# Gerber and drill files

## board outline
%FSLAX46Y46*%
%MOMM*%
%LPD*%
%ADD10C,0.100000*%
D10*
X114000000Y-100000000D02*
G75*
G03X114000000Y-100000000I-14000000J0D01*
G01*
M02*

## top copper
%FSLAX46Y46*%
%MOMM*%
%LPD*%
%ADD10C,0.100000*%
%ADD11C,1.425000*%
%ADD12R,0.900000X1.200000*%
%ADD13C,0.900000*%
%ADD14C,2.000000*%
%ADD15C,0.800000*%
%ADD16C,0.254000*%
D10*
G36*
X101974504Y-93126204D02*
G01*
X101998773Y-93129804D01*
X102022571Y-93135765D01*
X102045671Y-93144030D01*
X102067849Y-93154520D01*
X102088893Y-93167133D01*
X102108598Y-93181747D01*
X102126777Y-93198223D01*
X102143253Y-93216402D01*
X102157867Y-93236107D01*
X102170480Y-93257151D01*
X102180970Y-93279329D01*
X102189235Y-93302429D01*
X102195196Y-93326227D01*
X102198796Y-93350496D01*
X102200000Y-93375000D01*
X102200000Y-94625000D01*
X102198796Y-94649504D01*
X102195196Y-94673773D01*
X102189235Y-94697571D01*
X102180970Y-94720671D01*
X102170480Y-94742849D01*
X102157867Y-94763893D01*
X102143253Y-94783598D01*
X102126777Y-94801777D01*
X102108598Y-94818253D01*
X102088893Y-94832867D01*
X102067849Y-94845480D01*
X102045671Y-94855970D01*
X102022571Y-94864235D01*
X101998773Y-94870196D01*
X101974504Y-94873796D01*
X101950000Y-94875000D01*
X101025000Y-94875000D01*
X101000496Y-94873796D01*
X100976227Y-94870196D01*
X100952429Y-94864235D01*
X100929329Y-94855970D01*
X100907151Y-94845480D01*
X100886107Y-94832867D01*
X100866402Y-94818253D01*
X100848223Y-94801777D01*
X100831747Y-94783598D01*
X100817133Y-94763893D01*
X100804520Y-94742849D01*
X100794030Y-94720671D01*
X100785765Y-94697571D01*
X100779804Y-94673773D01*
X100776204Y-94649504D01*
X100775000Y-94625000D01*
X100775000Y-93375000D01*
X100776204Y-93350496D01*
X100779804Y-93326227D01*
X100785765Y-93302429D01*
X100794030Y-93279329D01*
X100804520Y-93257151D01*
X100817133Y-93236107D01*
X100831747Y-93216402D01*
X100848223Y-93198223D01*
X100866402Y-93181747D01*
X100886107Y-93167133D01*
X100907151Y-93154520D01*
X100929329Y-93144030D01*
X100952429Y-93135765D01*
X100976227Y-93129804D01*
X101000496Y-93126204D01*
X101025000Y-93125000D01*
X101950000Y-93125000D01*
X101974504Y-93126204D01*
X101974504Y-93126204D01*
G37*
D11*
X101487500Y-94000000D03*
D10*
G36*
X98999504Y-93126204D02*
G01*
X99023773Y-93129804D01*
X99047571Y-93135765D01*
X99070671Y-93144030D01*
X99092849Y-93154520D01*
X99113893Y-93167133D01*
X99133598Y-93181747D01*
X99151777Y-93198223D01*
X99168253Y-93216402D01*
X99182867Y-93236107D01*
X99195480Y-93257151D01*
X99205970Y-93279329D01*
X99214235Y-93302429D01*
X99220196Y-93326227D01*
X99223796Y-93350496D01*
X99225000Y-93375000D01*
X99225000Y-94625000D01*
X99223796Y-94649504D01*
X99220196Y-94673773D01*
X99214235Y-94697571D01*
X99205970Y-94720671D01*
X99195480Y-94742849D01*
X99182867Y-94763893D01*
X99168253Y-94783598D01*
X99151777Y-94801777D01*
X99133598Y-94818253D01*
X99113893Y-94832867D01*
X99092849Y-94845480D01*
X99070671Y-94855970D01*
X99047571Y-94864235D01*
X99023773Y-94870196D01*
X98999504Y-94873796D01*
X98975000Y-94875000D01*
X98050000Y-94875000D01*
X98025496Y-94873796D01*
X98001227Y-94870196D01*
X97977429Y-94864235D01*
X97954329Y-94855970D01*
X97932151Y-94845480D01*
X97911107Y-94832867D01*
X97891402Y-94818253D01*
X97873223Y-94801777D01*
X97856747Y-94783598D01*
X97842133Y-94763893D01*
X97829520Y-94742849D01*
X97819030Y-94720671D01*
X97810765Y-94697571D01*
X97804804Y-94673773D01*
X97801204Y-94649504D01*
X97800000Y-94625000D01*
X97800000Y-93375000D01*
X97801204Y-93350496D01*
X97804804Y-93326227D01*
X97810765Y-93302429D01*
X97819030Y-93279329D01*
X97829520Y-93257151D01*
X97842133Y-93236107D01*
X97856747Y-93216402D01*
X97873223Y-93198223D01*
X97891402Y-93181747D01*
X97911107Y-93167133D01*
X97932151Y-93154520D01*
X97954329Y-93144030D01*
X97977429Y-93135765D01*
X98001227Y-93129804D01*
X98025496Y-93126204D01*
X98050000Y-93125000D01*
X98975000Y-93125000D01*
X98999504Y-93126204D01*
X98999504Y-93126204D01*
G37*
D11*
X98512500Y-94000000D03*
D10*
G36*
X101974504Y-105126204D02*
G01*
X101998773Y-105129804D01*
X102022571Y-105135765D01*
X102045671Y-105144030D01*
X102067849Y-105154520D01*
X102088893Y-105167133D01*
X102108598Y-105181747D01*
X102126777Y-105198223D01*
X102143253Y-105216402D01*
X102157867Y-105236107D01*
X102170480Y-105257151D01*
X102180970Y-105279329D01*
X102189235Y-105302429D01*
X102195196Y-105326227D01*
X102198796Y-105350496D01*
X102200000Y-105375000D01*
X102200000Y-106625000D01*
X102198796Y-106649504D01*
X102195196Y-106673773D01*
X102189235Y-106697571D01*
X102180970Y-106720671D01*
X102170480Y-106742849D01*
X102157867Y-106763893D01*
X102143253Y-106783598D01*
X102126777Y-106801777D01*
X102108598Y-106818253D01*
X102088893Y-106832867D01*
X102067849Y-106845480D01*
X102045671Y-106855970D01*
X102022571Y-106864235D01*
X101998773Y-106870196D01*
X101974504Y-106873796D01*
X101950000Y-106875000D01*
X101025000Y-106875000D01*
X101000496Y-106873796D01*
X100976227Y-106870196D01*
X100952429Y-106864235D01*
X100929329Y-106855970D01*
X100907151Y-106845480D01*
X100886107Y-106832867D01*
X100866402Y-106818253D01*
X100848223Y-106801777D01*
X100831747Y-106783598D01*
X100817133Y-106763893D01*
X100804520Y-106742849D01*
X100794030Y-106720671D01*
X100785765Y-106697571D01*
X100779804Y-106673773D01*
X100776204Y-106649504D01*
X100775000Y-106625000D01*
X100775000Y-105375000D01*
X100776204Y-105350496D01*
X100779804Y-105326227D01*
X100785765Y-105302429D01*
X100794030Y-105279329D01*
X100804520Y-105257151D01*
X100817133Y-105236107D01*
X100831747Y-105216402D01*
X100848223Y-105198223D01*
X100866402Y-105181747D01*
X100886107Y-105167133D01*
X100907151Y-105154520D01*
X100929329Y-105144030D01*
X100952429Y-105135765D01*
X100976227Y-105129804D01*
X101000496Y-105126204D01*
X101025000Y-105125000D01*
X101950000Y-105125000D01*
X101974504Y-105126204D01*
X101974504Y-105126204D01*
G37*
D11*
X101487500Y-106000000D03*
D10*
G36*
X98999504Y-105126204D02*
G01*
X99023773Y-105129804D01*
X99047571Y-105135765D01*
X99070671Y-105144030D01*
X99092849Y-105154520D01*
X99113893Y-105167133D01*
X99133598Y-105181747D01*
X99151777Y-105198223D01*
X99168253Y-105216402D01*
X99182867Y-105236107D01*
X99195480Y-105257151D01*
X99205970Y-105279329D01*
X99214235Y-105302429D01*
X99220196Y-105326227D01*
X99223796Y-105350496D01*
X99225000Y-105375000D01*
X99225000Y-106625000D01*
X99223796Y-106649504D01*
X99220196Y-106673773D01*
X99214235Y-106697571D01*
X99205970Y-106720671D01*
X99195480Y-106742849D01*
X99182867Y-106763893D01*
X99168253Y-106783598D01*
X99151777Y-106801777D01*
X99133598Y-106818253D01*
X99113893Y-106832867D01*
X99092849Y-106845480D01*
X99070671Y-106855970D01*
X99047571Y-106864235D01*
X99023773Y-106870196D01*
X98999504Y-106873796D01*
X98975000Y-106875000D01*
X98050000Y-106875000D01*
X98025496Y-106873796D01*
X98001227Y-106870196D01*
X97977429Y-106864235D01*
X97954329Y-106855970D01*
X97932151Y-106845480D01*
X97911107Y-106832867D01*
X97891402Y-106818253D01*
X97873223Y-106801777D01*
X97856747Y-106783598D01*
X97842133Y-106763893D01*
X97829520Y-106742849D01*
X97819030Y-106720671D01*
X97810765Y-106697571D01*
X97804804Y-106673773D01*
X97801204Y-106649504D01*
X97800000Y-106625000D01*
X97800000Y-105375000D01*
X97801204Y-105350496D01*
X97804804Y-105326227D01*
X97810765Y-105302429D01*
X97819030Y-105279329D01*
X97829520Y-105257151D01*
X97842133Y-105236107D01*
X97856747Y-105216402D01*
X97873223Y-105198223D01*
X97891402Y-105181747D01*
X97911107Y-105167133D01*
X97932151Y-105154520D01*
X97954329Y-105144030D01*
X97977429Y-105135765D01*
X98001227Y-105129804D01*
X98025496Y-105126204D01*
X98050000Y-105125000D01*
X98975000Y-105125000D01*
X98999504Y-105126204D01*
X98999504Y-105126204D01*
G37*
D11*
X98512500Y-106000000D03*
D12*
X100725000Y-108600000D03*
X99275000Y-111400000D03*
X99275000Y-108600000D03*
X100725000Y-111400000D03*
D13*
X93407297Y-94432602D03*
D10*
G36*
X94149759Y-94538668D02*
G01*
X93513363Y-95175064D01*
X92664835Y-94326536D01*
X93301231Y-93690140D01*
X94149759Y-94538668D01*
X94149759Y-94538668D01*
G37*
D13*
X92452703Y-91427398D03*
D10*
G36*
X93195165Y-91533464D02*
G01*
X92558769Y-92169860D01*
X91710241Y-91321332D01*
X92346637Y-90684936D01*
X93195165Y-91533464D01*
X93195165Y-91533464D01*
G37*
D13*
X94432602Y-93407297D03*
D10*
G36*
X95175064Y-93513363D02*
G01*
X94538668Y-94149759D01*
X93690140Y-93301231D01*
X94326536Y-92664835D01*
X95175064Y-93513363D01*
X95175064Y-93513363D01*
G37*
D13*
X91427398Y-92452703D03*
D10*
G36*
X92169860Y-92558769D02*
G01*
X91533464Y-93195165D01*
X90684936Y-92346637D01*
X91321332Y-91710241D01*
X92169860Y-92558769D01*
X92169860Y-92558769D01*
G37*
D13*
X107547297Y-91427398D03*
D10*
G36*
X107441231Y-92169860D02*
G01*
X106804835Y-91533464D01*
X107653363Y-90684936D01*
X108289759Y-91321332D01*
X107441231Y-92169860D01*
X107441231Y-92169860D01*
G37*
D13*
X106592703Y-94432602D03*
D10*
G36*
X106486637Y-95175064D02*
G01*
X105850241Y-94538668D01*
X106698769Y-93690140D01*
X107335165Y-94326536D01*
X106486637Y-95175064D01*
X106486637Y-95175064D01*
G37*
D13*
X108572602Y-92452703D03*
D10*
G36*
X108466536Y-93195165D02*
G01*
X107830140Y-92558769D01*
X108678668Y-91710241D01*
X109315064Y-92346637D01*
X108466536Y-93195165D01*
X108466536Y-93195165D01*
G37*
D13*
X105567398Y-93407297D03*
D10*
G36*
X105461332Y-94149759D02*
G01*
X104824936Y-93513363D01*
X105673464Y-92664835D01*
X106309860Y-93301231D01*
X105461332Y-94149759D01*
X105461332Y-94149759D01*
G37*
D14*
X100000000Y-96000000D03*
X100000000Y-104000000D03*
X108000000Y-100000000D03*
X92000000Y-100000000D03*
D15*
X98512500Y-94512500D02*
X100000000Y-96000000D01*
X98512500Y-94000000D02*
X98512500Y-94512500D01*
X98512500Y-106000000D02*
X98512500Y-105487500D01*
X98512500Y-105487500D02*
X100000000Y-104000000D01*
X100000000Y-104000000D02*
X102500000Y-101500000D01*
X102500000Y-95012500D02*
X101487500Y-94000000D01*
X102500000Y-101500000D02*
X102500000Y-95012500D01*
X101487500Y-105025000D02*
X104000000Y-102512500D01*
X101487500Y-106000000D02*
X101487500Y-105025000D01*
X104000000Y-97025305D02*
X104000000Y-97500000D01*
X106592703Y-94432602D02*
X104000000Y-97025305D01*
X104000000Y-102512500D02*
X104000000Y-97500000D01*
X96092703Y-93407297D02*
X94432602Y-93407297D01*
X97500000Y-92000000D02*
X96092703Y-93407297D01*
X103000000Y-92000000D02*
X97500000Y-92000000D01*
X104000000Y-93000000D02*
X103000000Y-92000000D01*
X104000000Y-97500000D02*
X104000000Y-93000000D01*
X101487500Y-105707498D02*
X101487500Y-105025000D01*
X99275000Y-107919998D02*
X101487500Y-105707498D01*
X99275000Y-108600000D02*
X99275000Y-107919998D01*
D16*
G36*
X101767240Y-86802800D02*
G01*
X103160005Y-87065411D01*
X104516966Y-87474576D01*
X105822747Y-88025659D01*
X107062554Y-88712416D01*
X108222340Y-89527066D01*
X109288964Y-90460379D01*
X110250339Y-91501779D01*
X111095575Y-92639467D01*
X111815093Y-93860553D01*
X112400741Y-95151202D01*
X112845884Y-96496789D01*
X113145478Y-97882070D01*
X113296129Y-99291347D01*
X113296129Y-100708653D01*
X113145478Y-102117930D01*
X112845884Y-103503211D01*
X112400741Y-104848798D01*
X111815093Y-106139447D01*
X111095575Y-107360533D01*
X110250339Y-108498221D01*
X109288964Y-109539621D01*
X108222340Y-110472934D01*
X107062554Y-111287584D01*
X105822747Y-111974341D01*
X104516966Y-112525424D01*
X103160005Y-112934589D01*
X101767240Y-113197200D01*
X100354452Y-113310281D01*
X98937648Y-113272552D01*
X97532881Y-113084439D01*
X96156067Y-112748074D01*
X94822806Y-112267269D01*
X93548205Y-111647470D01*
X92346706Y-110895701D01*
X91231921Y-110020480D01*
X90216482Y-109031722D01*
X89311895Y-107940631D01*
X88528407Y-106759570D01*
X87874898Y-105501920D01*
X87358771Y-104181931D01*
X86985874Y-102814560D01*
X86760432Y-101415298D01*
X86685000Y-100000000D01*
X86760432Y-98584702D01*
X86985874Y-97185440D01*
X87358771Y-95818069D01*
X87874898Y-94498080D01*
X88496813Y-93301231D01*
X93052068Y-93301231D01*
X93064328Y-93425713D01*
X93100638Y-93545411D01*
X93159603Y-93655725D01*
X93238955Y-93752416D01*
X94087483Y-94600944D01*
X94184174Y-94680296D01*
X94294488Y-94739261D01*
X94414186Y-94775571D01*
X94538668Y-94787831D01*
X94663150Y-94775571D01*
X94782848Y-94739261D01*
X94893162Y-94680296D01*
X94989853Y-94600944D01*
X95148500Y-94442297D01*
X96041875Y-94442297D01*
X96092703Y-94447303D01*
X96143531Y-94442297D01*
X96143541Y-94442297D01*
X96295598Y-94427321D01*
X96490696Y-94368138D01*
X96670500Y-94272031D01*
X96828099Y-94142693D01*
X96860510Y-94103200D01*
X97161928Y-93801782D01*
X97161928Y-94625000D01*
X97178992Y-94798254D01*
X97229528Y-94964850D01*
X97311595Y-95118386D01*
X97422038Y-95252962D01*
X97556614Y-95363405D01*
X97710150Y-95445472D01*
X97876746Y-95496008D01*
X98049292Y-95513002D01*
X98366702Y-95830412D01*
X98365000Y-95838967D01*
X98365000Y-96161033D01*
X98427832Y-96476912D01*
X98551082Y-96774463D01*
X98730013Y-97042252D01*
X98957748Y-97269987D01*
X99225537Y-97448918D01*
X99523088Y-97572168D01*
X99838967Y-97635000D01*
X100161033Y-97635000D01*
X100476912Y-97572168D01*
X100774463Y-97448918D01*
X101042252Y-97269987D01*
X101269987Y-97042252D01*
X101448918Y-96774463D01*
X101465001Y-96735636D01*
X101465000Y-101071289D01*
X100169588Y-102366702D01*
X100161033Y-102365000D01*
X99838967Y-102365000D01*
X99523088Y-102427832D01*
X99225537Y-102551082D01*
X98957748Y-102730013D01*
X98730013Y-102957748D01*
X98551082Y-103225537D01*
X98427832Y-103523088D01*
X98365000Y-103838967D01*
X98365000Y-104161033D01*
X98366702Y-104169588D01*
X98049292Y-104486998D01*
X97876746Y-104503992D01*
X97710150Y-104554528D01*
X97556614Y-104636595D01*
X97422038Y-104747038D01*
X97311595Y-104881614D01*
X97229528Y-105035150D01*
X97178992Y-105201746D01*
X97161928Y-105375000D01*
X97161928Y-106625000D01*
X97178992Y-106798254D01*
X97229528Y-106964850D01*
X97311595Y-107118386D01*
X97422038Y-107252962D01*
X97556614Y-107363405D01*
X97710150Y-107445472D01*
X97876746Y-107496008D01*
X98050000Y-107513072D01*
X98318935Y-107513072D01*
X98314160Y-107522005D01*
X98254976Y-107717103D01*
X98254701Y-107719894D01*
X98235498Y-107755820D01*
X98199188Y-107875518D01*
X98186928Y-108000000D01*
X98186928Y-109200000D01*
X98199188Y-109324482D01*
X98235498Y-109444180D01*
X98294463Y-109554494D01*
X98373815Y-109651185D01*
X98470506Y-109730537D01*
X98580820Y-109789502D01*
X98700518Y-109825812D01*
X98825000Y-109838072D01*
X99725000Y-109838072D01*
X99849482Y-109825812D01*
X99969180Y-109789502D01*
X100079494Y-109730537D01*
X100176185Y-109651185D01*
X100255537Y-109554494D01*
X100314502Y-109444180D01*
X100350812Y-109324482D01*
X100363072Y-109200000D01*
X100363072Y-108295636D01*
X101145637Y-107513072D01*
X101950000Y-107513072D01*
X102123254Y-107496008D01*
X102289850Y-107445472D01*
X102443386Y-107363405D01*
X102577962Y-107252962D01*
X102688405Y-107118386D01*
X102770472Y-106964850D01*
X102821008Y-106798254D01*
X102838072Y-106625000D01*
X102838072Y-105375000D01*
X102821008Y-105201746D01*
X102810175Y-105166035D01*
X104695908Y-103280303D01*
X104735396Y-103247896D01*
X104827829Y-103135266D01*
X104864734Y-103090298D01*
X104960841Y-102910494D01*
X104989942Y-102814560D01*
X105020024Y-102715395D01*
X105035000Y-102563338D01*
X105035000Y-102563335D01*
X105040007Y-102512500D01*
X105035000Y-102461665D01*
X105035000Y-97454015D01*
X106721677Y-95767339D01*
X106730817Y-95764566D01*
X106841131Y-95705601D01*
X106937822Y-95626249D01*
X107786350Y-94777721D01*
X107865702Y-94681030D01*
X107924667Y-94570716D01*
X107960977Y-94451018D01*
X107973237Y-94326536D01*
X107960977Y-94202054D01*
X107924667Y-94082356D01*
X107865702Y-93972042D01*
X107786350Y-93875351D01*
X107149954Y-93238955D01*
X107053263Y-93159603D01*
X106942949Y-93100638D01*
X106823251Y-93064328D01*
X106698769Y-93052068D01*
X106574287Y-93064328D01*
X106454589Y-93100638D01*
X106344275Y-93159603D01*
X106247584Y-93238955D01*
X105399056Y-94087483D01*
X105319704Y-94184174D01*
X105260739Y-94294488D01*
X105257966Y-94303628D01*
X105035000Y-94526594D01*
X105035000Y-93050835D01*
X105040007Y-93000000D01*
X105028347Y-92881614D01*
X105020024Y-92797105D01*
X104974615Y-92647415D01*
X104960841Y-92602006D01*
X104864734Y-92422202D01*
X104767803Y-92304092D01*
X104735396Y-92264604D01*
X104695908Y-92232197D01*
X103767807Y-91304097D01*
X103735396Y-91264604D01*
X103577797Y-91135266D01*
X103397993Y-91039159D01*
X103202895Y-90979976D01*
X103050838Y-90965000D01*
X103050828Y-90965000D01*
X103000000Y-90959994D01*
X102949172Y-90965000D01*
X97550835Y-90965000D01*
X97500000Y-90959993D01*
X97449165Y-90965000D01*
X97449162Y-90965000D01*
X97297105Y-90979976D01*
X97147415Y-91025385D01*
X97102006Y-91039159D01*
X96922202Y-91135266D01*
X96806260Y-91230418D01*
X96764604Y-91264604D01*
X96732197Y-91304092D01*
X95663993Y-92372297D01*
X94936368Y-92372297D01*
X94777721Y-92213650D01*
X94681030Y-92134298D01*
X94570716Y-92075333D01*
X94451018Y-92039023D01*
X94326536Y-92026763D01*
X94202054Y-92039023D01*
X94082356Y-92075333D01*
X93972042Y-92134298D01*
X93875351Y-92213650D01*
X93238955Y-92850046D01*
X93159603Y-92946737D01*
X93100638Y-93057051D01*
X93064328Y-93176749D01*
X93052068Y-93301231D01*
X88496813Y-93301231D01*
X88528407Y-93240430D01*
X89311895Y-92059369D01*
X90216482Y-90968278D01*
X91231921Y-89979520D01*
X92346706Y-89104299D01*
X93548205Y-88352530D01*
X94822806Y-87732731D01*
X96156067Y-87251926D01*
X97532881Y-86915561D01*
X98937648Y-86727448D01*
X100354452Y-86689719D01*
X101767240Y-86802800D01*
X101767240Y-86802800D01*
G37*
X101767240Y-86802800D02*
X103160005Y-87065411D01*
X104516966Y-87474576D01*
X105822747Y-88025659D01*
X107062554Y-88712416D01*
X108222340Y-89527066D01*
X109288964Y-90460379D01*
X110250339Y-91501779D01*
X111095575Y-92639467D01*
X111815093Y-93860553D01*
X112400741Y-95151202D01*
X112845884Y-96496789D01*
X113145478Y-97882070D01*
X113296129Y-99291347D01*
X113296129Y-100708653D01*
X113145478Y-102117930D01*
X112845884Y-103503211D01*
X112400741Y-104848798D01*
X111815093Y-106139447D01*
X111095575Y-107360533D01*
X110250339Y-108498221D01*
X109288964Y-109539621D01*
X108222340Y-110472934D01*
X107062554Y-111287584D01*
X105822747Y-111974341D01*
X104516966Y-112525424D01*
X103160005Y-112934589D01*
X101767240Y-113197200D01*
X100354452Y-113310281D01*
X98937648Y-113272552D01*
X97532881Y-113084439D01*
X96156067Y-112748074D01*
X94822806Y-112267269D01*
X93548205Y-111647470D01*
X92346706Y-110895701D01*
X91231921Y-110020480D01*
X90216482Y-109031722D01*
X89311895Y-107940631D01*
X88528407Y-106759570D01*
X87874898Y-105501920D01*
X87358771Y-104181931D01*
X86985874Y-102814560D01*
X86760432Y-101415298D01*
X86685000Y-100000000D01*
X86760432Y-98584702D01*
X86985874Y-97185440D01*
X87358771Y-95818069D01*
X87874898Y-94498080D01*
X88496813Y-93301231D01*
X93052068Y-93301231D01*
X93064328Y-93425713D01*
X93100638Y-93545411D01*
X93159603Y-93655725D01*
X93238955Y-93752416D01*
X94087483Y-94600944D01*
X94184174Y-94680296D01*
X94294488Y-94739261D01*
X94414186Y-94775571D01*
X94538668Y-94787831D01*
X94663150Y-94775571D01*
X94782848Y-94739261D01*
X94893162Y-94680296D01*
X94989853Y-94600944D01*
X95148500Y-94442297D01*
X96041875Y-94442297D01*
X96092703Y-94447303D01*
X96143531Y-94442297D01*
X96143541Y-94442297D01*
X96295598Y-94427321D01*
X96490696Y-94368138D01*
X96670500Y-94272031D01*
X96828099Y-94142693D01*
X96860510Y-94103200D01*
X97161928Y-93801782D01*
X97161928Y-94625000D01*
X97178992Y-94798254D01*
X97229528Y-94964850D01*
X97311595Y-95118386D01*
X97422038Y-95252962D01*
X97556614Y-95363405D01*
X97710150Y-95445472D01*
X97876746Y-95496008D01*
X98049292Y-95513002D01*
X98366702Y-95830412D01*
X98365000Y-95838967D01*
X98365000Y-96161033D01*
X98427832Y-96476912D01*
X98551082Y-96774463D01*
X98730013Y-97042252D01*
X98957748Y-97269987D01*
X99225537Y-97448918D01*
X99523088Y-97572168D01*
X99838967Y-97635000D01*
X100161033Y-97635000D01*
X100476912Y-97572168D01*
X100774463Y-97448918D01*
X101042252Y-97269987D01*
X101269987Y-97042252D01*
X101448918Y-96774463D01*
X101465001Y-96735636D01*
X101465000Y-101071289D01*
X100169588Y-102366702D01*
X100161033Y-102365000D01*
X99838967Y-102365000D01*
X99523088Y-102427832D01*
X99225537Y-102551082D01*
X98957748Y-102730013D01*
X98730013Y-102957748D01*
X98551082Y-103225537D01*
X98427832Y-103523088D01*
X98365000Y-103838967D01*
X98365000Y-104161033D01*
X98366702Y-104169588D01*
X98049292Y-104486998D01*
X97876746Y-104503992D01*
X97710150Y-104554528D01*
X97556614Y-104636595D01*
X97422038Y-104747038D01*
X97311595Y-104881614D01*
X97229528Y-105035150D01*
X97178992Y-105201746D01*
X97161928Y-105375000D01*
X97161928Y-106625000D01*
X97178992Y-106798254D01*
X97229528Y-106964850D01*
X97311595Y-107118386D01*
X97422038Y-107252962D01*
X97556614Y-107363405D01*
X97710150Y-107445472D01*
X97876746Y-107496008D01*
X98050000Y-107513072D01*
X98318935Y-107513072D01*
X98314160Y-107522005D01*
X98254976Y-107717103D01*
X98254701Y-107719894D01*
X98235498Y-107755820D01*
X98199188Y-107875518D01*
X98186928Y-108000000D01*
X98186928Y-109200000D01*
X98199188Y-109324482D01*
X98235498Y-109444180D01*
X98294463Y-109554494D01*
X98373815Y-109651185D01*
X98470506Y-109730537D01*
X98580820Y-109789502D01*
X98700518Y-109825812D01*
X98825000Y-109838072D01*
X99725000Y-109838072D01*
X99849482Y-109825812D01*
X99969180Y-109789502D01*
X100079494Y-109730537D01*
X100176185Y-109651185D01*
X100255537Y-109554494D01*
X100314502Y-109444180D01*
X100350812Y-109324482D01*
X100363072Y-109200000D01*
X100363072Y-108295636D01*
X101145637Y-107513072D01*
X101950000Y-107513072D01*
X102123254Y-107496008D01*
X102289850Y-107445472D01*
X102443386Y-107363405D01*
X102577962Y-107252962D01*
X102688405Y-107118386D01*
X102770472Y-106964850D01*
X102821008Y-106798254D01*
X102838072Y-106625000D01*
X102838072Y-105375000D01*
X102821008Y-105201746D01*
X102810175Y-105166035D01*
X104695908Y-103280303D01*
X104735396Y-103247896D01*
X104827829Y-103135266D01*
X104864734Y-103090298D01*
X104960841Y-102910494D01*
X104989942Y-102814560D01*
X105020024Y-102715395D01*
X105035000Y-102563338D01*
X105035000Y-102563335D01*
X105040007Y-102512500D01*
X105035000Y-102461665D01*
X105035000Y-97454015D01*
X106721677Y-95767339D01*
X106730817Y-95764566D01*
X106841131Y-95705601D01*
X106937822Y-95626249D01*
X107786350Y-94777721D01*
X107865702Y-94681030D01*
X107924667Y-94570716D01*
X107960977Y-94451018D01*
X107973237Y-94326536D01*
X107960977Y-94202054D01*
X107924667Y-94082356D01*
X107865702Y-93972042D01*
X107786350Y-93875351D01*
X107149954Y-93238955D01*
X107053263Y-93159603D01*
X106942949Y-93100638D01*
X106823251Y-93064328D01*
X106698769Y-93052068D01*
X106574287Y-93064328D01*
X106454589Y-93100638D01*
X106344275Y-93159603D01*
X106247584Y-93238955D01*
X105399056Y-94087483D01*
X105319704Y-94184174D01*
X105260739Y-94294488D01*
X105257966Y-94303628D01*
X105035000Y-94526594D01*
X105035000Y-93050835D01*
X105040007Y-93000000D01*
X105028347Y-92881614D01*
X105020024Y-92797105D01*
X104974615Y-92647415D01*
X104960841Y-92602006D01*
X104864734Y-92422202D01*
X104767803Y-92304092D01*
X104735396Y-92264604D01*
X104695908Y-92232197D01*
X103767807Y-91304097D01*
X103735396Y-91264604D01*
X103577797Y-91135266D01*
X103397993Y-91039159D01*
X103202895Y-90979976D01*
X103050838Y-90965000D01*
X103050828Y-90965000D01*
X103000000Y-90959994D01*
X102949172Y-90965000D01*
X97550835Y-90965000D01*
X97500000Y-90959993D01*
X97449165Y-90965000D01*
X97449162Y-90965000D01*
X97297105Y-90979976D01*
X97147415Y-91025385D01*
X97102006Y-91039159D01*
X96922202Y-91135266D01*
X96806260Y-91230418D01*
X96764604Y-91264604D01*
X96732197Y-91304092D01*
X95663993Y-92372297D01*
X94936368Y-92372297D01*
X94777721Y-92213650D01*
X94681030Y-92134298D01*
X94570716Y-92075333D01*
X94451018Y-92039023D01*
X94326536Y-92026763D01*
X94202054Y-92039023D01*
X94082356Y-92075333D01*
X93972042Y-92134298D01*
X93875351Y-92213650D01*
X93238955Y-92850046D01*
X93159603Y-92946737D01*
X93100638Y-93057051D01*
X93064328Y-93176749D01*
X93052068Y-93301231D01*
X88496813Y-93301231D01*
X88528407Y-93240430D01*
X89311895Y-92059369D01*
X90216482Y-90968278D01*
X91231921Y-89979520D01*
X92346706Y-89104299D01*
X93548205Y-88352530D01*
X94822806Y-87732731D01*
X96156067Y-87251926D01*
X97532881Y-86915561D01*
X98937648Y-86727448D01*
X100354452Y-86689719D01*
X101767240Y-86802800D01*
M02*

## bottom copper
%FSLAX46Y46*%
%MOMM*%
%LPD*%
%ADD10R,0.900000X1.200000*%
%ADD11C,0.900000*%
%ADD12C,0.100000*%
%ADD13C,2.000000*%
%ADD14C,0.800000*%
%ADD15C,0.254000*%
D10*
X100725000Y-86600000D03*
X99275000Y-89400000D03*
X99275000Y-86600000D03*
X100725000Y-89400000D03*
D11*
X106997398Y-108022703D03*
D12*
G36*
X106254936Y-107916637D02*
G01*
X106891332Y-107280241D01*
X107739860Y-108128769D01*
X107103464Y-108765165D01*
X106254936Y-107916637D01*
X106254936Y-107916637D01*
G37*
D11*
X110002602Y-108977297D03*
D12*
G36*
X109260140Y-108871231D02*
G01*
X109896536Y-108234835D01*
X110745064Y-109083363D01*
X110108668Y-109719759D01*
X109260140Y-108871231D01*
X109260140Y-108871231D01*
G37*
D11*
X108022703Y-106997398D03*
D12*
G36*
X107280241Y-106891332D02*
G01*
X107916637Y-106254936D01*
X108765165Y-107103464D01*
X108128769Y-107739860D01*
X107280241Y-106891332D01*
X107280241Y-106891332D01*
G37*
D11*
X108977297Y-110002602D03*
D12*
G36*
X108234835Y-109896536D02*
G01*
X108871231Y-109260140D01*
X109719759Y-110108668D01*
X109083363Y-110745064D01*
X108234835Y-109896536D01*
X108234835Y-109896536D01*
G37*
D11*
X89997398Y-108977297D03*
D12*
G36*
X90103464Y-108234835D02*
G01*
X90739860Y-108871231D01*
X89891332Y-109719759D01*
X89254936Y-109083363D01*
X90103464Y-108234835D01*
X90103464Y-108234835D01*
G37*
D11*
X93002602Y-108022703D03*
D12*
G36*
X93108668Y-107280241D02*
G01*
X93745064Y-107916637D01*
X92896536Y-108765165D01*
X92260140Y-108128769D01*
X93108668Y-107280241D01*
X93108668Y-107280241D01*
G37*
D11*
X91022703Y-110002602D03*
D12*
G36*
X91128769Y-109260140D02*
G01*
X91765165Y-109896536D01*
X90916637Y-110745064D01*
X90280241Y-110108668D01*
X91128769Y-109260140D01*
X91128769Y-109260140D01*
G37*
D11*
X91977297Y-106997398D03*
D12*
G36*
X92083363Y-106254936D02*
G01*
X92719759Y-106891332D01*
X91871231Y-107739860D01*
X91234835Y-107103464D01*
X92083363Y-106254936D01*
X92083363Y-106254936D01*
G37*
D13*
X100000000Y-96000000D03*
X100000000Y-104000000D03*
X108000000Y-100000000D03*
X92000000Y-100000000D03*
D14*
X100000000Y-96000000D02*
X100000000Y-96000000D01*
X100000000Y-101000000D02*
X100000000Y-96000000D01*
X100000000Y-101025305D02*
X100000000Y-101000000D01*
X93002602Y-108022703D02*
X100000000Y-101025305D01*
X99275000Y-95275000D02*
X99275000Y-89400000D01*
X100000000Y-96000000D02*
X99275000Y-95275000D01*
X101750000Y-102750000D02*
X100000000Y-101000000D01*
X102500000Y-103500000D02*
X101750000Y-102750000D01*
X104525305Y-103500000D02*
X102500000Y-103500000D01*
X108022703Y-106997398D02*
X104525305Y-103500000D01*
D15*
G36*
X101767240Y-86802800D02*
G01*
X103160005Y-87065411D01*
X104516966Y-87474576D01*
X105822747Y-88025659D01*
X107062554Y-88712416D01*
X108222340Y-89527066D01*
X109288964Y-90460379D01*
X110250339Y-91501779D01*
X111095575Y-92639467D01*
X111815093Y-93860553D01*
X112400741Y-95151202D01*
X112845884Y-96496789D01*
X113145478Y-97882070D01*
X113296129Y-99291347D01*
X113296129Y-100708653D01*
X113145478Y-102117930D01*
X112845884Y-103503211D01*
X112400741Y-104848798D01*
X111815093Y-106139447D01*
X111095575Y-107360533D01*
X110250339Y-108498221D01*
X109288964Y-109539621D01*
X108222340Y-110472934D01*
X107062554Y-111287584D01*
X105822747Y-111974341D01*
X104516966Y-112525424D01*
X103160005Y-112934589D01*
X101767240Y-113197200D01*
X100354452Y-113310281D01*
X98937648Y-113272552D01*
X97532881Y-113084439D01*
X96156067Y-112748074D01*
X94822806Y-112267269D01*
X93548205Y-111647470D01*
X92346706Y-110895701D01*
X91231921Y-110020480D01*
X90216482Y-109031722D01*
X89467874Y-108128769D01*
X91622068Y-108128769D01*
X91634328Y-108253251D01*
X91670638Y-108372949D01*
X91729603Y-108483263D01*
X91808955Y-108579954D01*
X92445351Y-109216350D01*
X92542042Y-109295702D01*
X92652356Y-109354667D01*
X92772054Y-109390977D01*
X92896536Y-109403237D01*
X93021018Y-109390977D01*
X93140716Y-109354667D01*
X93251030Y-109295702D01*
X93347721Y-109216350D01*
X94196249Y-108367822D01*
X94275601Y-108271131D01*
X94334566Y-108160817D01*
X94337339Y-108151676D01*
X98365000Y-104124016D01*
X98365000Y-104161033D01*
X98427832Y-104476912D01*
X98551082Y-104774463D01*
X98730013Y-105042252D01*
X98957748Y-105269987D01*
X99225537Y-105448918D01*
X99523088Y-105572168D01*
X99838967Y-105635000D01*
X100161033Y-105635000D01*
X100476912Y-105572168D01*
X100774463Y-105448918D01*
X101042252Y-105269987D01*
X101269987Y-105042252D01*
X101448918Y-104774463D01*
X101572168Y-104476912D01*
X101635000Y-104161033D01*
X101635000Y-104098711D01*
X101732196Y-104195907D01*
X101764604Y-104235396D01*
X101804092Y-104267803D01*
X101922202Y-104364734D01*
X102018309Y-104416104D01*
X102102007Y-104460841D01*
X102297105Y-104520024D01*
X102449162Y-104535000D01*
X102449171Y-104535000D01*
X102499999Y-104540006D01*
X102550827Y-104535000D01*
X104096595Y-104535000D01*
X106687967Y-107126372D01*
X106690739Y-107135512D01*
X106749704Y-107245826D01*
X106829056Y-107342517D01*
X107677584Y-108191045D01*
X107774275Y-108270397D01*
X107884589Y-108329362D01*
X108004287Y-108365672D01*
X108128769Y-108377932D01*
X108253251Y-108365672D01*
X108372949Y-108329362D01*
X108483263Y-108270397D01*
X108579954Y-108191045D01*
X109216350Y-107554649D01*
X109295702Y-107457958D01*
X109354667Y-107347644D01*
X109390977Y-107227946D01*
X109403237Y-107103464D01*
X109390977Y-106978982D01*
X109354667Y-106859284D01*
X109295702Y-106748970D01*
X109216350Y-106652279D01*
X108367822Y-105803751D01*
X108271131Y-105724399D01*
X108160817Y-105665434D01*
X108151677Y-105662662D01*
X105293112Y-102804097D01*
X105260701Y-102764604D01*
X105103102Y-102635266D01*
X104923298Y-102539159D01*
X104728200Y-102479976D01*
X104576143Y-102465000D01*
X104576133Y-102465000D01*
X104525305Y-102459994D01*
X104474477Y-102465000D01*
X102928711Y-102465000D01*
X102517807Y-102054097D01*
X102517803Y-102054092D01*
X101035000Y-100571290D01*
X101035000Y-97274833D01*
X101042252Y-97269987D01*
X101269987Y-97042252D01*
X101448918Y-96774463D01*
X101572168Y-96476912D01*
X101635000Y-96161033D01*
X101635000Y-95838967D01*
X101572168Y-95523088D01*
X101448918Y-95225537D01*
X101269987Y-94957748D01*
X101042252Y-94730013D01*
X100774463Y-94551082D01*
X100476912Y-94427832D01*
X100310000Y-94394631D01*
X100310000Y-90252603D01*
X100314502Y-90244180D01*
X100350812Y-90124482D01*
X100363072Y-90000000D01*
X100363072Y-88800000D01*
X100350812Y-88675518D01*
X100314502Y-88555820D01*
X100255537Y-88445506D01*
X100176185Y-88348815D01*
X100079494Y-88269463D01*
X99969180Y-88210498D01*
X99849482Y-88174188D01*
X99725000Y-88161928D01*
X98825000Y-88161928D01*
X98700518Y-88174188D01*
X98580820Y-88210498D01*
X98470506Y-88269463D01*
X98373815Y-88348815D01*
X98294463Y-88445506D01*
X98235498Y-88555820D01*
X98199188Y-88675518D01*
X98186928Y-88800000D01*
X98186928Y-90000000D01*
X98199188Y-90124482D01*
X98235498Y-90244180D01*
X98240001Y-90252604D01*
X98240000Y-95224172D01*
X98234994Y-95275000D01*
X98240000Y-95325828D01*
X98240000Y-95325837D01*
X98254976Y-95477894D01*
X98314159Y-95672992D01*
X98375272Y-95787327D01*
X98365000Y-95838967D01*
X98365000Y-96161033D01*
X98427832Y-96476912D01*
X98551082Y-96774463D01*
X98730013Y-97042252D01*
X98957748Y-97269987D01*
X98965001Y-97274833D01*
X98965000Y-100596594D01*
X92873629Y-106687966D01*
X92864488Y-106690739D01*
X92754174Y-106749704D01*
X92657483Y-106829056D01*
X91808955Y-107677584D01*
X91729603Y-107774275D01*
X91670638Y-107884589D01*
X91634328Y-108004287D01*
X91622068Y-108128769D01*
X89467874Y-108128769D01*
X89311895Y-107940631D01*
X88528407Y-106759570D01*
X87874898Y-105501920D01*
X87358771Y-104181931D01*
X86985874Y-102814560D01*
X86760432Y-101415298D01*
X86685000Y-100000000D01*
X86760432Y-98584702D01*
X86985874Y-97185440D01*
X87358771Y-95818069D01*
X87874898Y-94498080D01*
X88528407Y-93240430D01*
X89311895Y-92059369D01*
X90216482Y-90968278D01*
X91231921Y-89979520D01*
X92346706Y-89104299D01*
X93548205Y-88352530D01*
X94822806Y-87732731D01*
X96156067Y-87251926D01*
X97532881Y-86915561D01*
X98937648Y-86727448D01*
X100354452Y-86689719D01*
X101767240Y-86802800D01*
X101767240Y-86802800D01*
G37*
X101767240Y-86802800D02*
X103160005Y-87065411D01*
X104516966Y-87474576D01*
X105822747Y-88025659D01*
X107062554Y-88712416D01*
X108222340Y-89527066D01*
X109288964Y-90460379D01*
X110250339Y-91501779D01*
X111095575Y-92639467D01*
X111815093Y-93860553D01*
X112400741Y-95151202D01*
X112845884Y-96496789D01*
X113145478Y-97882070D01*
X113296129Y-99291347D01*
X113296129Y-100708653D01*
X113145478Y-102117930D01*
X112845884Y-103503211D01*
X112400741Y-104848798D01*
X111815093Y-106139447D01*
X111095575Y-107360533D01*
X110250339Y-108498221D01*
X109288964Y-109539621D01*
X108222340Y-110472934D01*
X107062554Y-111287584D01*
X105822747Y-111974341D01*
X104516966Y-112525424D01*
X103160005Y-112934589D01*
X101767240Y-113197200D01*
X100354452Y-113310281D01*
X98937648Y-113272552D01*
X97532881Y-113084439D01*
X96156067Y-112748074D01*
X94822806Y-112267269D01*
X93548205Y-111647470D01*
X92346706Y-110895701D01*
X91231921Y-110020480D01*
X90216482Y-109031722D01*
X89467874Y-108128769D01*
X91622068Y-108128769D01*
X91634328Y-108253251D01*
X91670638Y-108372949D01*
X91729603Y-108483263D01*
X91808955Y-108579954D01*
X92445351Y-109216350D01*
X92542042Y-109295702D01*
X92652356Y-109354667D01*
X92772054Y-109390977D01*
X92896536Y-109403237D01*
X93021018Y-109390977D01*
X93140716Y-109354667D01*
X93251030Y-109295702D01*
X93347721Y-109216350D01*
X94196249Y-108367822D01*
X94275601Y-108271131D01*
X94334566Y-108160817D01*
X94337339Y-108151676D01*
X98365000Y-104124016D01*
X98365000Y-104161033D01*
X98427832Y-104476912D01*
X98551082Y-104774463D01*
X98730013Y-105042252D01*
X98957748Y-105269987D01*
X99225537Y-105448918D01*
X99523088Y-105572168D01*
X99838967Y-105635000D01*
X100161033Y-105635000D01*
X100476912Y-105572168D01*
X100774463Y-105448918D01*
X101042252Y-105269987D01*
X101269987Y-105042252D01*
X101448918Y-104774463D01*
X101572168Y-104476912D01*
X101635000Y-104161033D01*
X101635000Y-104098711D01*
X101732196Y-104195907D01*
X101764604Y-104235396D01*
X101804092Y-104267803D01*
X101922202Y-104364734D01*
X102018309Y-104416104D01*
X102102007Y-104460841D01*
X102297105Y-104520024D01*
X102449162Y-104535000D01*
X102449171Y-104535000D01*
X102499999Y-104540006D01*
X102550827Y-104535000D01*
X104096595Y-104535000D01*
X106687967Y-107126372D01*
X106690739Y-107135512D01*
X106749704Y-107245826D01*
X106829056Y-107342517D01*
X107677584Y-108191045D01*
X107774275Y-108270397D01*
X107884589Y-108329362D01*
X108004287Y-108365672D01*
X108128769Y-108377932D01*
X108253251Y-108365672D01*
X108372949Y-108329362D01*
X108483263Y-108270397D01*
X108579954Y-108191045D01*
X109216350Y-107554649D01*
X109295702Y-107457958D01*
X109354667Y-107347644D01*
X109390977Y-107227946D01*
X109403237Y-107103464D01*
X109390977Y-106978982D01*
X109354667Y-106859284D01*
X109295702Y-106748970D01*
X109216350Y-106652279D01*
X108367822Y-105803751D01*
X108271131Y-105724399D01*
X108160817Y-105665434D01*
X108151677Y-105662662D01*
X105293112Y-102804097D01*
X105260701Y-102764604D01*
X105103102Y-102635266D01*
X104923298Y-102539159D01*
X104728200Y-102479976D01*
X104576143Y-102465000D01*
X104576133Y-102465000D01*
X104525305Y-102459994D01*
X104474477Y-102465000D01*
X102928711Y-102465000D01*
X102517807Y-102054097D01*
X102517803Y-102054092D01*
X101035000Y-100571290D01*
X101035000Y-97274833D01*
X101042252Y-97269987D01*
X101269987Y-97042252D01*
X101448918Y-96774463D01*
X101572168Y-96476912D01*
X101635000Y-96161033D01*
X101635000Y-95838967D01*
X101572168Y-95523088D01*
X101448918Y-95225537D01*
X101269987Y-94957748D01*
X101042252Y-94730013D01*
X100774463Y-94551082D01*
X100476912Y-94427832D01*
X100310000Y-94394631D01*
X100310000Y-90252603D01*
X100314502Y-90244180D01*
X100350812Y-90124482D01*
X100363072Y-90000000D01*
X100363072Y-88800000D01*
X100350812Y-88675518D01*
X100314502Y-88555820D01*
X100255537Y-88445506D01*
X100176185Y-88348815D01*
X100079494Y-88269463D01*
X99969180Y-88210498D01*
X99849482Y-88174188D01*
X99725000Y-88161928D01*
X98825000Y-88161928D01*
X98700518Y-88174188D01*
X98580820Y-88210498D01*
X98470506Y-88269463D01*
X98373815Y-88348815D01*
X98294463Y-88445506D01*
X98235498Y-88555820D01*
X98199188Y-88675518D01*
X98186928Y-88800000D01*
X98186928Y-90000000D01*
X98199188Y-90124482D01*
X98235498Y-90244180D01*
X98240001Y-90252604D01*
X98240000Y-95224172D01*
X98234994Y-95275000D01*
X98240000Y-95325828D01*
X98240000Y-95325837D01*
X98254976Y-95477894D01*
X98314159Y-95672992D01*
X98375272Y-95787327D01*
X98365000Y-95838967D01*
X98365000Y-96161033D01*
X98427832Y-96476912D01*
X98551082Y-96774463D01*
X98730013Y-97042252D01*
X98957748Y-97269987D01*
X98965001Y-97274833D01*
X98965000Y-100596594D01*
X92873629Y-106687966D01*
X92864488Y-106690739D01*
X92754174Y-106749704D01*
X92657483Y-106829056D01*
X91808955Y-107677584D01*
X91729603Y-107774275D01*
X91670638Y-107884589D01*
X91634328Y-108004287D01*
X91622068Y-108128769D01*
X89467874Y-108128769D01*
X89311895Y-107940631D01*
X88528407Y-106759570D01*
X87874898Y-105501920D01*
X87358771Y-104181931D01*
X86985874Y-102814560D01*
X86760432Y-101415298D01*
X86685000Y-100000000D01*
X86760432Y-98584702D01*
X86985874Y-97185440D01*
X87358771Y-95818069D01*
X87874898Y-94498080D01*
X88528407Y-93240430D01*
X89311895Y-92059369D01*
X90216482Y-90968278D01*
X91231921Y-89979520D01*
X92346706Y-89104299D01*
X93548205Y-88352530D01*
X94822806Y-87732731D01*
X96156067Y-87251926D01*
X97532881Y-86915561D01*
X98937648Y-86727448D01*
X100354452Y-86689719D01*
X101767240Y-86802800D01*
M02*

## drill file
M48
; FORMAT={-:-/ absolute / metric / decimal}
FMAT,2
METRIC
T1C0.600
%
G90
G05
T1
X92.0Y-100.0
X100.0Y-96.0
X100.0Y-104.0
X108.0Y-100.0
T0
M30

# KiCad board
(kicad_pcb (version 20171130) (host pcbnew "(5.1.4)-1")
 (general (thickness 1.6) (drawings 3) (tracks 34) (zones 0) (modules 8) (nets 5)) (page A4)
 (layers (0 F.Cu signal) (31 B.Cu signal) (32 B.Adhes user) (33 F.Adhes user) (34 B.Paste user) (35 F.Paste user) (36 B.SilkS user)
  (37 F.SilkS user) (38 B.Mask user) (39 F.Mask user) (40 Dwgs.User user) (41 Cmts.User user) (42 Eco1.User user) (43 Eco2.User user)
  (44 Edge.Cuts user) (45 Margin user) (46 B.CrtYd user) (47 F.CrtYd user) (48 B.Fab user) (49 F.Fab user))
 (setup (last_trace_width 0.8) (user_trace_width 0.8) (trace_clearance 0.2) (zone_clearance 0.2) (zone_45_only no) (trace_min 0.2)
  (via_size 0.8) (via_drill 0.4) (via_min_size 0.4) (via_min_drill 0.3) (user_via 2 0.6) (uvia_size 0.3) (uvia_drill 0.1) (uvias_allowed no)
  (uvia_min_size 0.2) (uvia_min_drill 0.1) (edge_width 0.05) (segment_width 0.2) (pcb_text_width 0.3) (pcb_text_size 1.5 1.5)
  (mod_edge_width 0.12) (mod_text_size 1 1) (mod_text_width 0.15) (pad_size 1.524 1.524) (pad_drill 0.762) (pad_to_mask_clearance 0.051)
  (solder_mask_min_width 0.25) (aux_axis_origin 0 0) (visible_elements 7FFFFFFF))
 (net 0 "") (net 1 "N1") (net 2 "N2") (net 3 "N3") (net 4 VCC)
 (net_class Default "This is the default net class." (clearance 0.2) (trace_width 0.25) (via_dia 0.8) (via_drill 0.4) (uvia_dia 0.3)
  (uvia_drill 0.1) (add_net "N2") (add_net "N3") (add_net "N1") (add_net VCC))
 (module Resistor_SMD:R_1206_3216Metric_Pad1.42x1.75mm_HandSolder (layer F.Cu) (at 100 94 180)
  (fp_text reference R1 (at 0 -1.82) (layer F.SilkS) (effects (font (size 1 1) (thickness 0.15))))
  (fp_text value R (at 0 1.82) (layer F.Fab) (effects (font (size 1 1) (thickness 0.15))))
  (pad 1 smd roundrect (at -1.4875 0 180) (size 1.425 1.75) (layers F.Cu F.Paste F.Mask) (roundrect_rratio 0.175439) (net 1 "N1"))
  (pad 2 smd roundrect (at 1.4875 0 180) (size 1.425 1.75) (layers F.Cu F.Paste F.Mask) (roundrect_rratio 0.175439) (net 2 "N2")))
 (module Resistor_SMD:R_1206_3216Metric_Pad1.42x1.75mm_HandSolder (layer F.Cu) (at 100 106)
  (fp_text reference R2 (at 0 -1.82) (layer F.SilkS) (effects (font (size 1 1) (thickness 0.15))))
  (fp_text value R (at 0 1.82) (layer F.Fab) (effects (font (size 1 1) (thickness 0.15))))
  (pad 2 smd roundrect (at 1.4875 0) (size 1.425 1.75) (layers F.Cu F.Paste F.Mask) (roundrect_rratio 0.175439) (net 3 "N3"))
  (pad 1 smd roundrect (at -1.4875 0) (size 1.425 1.75) (layers F.Cu F.Paste F.Mask) (roundrect_rratio 0.175439) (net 1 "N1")))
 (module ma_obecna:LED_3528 (layer B.Cu) (at 100 88 90)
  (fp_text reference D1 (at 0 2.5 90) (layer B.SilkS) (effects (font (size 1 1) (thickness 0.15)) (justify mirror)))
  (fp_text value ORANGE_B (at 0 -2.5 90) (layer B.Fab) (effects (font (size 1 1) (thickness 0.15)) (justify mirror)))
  (pad 3 smd rect (at 1.4 0.725 90) (size 1.2 0.9) (layers B.Cu B.Paste B.Mask) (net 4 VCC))
  (pad 1 smd rect (at -1.4 -0.725 90) (size 1.2 0.9) (layers B.Cu B.Paste B.Mask) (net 2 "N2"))
  (pad 2 smd rect (at 1.4 -0.725 90) (size 1.2 0.9) (layers B.Cu B.Paste B.Mask) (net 4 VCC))
  (pad 4 smd rect (at -1.4 0.725 90) (size 1.2 0.9) (layers B.Cu B.Paste B.Mask) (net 4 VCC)))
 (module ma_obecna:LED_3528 (layer B.Cu) (at 108.5 108.5 315)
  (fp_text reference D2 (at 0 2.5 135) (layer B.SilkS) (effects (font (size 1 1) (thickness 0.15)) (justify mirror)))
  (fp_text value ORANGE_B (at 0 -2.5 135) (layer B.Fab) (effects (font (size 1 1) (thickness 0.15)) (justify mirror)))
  (pad 4 smd rect (at -1.4 0.725 315) (size 1.2 0.9) (layers B.Cu B.Paste B.Mask) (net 4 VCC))
  (pad 2 smd rect (at 1.4 -0.725 315) (size 1.2 0.9) (layers B.Cu B.Paste B.Mask) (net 4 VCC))
  (pad 1 smd rect (at -1.4 -0.725 315) (size 1.2 0.9) (layers B.Cu B.Paste B.Mask) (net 2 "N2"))
  (pad 3 smd rect (at 1.4 0.725 315) (size 1.2 0.9) (layers B.Cu B.Paste B.Mask) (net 4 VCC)))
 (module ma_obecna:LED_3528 (layer B.Cu) (at 91.5 108.5 225)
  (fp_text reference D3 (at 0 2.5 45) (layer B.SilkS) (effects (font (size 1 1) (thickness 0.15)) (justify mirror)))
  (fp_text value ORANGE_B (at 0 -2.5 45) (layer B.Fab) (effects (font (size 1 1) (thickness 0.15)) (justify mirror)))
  (pad 3 smd rect (at 1.4 0.725 225) (size 1.2 0.9) (layers B.Cu B.Paste B.Mask) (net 4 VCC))
  (pad 1 smd rect (at -1.4 -0.725 225) (size 1.2 0.9) (layers B.Cu B.Paste B.Mask) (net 2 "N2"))
  (pad 2 smd rect (at 1.4 -0.725 225) (size 1.2 0.9) (layers B.Cu B.Paste B.Mask) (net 4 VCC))
  (pad 4 smd rect (at -1.4 0.725 225) (size 1.2 0.9) (layers B.Cu B.Paste B.Mask) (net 4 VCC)))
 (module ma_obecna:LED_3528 (layer F.Cu) (at 100 110 270)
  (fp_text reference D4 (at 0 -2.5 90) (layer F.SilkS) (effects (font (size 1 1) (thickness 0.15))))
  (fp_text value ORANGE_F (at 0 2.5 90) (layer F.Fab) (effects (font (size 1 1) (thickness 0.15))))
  (pad 4 smd rect (at -1.4 -0.725 270) (size 1.2 0.9) (layers F.Cu F.Paste F.Mask) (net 4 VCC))
  (pad 2 smd rect (at 1.4 0.725 270) (size 1.2 0.9) (layers F.Cu F.Paste F.Mask) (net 4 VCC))
  (pad 1 smd rect (at -1.4 0.725 270) (size 1.2 0.9) (layers F.Cu F.Paste F.Mask) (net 3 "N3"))
  (pad 3 smd rect (at 1.4 -0.725 270) (size 1.2 0.9) (layers F.Cu F.Paste F.Mask) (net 4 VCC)))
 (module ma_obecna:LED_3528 (layer F.Cu) (at 92.93 92.93 135)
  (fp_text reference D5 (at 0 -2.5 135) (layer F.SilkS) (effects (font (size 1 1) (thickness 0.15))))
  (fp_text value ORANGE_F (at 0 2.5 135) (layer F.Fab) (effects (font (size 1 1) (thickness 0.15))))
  (pad 4 smd rect (at -1.4 -0.725 135) (size 1.2 0.9) (layers F.Cu F.Paste F.Mask) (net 4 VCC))
  (pad 2 smd rect (at 1.4 0.725 135) (size 1.2 0.9) (layers F.Cu F.Paste F.Mask) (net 4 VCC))
  (pad 1 smd rect (at -1.4 0.725 135) (size 1.2 0.9) (layers F.Cu F.Paste F.Mask) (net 3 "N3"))
  (pad 3 smd rect (at 1.4 -0.725 135) (size 1.2 0.9) (layers F.Cu F.Paste F.Mask) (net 4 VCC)))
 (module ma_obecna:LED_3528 (layer F.Cu) (at 107.07 92.93 45)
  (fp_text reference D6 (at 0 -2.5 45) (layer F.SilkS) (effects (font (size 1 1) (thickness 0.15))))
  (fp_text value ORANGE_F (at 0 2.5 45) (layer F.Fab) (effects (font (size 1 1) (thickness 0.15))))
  (pad 3 smd rect (at 1.4 -0.725 45) (size 1.2 0.9) (layers F.Cu F.Paste F.Mask) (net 4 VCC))
  (pad 1 smd rect (at -1.4 0.725 45) (size 1.2 0.9) (layers F.Cu F.Paste F.Mask) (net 3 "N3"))
  (pad 2 smd rect (at 1.4 0.725 45) (size 1.2 0.9) (layers F.Cu F.Paste F.Mask) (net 4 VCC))
  (pad 4 smd rect (at -1.4 -0.725 45) (size 1.2 0.9) (layers F.Cu F.Paste F.Mask) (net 4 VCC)))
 (gr_circle (center 100 100) (end 114 100) (layer Edge.Cuts) (width 0.1))
 (segment (start 100 96) (end 100 96) (width 0.8) (layer B.Cu) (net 2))
 (via (at 100 96) (size 2) (drill 0.6) (layers F.Cu B.Cu) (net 2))
 (segment (start 98.5125 94.5125) (end 100 96) (width 0.8) (layer F.Cu) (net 2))
 (segment (start 98.5125 94) (end 98.5125 94.5125) (width 0.8) (layer F.Cu) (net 2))
 (segment (start 100 101) (end 100 96) (width 0.8) (layer B.Cu) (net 2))
 (segment (start 100 101.025305) (end 100 101) (width 0.8) (layer B.Cu) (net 2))
 (segment (start 93.002602 108.022703) (end 100 101.025305) (width 0.8) (layer B.Cu) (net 2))
 (segment (start 99.275 95.275) (end 99.275 89.4) (width 0.8) (layer B.Cu) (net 2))
 (segment (start 100 96) (end 99.275 95.275) (width 0.8) (layer B.Cu) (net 2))
 (segment (start 101.75 102.75) (end 100 101) (width 0.8) (layer B.Cu) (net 2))
 (segment (start 102.5 103.5) (end 101.75 102.75) (width 0.8) (layer B.Cu) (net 2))
 (segment (start 104.525305 103.5) (end 102.5 103.5) (width 0.8) (layer B.Cu) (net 2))
 (segment (start 108.022703 106.997398) (end 104.525305 103.5) (width 0.8) (layer B.Cu) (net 2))
 (via (at 100 104) (size 2) (drill 0.6) (layers F.Cu B.Cu) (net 1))
 (segment (start 98.5125 106) (end 98.5125 105.4875) (width 0.8) (layer F.Cu) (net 1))
 (segment (start 98.5125 105.4875) (end 100 104) (width 0.8) (layer F.Cu) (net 1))
 (segment (start 100 104) (end 102.5 101.5) (width 0.8) (layer F.Cu) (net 1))
 (segment (start 102.5 95.0125) (end 101.4875 94) (width 0.8) (layer F.Cu) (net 1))
 (segment (start 102.5 101.5) (end 102.5 95.0125) (width 0.8) (layer F.Cu) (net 1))
 (via (at 108 100) (size 2) (drill 0.6) (layers F.Cu B.Cu) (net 4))
 (via (at 92 100) (size 2) (drill 0.6) (layers F.Cu B.Cu) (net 4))
 (segment (start 101.4875 105.025) (end 104 102.5125) (width 0.8) (layer F.Cu) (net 3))
 (segment (start 101.4875 106) (end 101.4875 105.025) (width 0.8) (layer F.Cu) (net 3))
 (segment (start 104 97.025305) (end 104 97.5) (width 0.8) (layer F.Cu) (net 3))
 (segment (start 106.592703 94.432602) (end 104 97.025305) (width 0.8) (layer F.Cu) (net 3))
 (segment (start 104 102.5125) (end 104 97.5) (width 0.8) (layer F.Cu) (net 3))
 (segment (start 96.092703 93.407297) (end 94.432602 93.407297) (width 0.8) (layer F.Cu) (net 3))
 (segment (start 97.5 92) (end 96.092703 93.407297) (width 0.8) (layer F.Cu) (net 3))
 (segment (start 103 92) (end 97.5 92) (width 0.8) (layer F.Cu) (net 3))
 (segment (start 104 93) (end 103 92) (width 0.8) (layer F.Cu) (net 3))
 (segment (start 104 97.5) (end 104 93) (width 0.8) (layer F.Cu) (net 3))
 (segment (start 101.4875 105.707498) (end 101.4875 105.025) (width 0.8) (layer F.Cu) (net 3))
 (segment (start 99.275 107.919998) (end 101.4875 105.707498) (width 0.8) (layer F.Cu) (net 3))
 (segment (start 99.275 108.6) (end 99.275 107.919998) (width 0.8) (layer F.Cu) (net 3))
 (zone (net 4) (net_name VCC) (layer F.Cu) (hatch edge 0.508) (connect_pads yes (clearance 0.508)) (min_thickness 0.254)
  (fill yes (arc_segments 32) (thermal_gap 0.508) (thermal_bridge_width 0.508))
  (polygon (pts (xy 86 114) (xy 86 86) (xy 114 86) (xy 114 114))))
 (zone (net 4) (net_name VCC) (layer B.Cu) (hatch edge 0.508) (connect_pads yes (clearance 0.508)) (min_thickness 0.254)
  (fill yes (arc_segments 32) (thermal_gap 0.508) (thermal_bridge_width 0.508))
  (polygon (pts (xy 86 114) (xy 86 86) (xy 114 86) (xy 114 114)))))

